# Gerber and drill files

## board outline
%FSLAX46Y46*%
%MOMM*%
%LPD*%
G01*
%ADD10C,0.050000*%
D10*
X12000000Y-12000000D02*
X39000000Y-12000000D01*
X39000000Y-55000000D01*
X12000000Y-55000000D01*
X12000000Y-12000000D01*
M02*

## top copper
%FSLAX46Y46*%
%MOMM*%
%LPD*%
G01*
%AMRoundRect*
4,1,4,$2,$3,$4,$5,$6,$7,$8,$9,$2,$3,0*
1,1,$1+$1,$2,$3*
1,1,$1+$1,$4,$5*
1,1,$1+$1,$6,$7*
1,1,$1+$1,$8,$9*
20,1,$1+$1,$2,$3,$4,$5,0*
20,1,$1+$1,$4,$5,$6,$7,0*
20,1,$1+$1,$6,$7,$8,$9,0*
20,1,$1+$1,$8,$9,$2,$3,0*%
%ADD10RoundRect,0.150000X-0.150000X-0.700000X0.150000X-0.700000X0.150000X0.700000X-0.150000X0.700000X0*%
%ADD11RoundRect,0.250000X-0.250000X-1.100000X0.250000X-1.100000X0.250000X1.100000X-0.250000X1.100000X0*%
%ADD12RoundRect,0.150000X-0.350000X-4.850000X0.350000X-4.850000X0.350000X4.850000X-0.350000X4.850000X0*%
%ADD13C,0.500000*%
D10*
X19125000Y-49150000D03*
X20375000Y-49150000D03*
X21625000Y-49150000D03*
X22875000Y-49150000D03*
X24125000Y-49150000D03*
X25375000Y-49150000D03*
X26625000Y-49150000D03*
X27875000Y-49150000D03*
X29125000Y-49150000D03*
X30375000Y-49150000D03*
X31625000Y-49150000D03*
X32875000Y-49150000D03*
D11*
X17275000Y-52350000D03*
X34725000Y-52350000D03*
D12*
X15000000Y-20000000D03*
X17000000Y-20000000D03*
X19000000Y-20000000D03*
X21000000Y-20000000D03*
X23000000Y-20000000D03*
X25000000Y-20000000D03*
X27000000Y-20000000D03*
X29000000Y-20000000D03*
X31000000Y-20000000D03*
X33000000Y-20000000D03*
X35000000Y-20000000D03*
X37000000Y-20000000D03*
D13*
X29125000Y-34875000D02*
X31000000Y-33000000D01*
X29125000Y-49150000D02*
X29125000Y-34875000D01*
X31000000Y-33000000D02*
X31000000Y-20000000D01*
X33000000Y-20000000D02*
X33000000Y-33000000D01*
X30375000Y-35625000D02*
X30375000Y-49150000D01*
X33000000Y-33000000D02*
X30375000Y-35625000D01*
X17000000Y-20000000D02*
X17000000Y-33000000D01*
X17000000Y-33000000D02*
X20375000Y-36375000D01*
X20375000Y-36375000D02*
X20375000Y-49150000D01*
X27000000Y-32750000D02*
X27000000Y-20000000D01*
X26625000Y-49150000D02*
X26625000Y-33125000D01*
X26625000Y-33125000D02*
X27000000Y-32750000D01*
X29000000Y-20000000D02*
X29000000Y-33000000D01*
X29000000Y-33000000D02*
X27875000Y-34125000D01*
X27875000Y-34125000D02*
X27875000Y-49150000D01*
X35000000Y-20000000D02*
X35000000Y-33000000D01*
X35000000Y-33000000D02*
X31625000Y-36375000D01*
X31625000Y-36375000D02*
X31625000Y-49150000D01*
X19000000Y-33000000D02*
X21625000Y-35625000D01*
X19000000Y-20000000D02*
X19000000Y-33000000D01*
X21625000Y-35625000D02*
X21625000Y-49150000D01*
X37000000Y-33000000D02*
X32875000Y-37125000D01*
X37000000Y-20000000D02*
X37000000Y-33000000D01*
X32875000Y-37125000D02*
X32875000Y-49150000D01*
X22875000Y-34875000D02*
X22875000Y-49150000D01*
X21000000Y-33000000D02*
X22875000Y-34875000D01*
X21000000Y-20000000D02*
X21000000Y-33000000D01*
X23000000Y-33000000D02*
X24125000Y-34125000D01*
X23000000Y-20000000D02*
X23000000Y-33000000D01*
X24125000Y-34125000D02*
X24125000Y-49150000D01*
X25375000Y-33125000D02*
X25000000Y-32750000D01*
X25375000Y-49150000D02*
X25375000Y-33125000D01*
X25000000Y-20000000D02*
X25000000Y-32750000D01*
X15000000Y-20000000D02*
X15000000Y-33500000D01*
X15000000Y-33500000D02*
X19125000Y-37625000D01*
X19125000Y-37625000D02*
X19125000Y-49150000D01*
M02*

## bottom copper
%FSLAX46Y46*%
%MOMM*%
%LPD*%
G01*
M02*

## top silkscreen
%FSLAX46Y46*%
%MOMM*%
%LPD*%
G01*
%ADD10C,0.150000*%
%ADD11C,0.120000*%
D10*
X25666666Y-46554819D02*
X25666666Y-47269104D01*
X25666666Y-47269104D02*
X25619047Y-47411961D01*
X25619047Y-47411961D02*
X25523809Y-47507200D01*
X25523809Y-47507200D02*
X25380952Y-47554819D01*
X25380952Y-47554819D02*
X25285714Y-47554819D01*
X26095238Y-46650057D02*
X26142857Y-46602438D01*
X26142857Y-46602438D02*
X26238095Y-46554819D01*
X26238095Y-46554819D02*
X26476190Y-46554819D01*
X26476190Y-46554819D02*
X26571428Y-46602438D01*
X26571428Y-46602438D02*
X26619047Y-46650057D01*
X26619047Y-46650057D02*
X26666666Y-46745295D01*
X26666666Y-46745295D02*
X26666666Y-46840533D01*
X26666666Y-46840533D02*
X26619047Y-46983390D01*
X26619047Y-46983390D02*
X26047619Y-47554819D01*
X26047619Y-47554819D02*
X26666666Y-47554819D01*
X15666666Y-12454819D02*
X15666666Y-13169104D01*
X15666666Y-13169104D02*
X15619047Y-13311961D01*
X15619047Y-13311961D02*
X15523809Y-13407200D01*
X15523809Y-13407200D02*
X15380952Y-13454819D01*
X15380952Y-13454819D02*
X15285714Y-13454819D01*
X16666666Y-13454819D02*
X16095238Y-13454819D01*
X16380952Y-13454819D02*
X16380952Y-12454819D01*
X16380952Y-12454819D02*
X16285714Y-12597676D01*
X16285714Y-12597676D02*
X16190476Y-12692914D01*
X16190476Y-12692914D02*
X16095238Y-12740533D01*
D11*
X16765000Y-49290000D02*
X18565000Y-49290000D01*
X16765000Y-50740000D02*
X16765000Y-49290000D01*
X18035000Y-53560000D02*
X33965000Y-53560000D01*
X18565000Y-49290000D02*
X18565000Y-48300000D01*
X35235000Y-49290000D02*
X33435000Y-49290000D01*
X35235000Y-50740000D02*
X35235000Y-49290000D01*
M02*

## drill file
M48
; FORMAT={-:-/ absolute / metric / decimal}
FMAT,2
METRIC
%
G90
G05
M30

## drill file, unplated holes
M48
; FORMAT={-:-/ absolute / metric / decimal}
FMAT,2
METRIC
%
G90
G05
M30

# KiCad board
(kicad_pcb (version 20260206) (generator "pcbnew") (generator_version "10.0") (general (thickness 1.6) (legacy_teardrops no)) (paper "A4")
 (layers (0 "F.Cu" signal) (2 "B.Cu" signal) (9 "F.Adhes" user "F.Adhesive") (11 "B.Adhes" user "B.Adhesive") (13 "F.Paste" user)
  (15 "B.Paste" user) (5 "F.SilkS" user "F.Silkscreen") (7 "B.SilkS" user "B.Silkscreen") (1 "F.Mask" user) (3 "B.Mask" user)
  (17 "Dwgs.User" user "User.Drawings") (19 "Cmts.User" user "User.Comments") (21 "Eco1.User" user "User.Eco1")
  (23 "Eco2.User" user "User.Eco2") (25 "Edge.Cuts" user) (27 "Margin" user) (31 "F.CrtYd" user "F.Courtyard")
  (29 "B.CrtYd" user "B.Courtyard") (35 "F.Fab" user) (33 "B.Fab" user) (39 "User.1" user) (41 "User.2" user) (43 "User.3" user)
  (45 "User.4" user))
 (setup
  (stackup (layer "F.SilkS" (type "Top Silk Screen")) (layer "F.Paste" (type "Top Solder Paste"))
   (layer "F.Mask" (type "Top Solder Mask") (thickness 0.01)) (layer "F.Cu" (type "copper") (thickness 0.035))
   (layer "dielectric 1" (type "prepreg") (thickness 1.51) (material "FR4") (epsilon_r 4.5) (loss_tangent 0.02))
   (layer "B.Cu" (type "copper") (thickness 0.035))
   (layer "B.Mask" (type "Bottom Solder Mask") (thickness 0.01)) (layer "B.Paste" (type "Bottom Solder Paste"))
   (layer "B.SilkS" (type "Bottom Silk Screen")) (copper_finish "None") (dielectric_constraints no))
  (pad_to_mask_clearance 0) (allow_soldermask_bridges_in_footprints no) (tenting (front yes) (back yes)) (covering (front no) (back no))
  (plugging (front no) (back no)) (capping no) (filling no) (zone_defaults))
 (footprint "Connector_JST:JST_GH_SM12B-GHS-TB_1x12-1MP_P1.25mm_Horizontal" (layer "F.Cu") (at 26 51)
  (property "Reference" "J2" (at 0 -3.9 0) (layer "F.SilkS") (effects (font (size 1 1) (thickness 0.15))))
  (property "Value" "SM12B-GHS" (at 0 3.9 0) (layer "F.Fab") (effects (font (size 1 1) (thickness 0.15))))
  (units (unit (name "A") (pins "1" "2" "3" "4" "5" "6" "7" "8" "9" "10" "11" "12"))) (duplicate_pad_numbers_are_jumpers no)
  (fp_line (start -9.235 -1.71) (end -7.435 -1.71) (stroke (width 0.12) (type solid)) (layer "F.SilkS"))
  (fp_line (start -9.235 -0.26) (end -9.235 -1.71) (stroke (width 0.12) (type solid)) (layer "F.SilkS"))
  (fp_line (start -7.965 2.56) (end 7.965 2.56) (stroke (width 0.12) (type solid)) (layer "F.SilkS"))
  (fp_line (start -7.435 -1.71) (end -7.435 -2.7) (stroke (width 0.12) (type solid)) (layer "F.SilkS"))
  (fp_line (start 9.235 -1.71) (end 7.435 -1.71) (stroke (width 0.12) (type solid)) (layer "F.SilkS"))
  (fp_line (start 9.235 -0.26) (end 9.235 -1.71) (stroke (width 0.12) (type solid)) (layer "F.SilkS"))
  (pad "1" smd roundrect (at -6.875 -1.85) (size 0.6 1.7) (layers "F.Cu" "F.Mask" "F.Paste") (roundrect_rratio 0.25) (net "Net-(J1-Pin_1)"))
  (pad "2" smd roundrect (at -5.625 -1.85) (size 0.6 1.7) (layers "F.Cu" "F.Mask" "F.Paste") (roundrect_rratio 0.25) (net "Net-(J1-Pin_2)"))
  (pad "3" smd roundrect (at -4.375 -1.85) (size 0.6 1.7) (layers "F.Cu" "F.Mask" "F.Paste") (roundrect_rratio 0.25) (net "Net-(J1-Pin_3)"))
  (pad "4" smd roundrect (at -3.125 -1.85) (size 0.6 1.7) (layers "F.Cu" "F.Mask" "F.Paste") (roundrect_rratio 0.25) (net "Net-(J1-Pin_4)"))
  (pad "5" smd roundrect (at -1.875 -1.85) (size 0.6 1.7) (layers "F.Cu" "F.Mask" "F.Paste") (roundrect_rratio 0.25) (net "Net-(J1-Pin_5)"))
  (pad "6" smd roundrect (at -0.625 -1.85) (size 0.6 1.7) (layers "F.Cu" "F.Mask" "F.Paste") (roundrect_rratio 0.25) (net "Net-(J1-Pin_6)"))
  (pad "7" smd roundrect (at 0.625 -1.85) (size 0.6 1.7) (layers "F.Cu" "F.Mask" "F.Paste") (roundrect_rratio 0.25) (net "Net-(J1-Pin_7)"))
  (pad "8" smd roundrect (at 1.875 -1.85) (size 0.6 1.7) (layers "F.Cu" "F.Mask" "F.Paste") (roundrect_rratio 0.25) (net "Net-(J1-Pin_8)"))
  (pad "9" smd roundrect (at 3.125 -1.85) (size 0.6 1.7) (layers "F.Cu" "F.Mask" "F.Paste") (roundrect_rratio 0.25) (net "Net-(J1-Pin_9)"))
  (pad "10" smd roundrect (at 4.375 -1.85) (size 0.6 1.7) (layers "F.Cu" "F.Mask" "F.Paste") (roundrect_rratio 0.25) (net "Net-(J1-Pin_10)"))
  (pad "11" smd roundrect (at 5.625 -1.85) (size 0.6 1.7) (layers "F.Cu" "F.Mask" "F.Paste") (roundrect_rratio 0.25) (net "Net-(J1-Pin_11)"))
  (pad "12" smd roundrect (at 6.875 -1.85) (size 0.6 1.7) (layers "F.Cu" "F.Mask" "F.Paste") (roundrect_rratio 0.25) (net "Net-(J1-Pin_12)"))
  (pad "MP" smd roundrect (at -8.725 1.35) (size 1 2.7) (layers "F.Cu" "F.Mask" "F.Paste") (roundrect_rratio 0.25))
  (pad "MP" smd roundrect (at 8.725 1.35) (size 1 2.7) (layers "F.Cu" "F.Mask" "F.Paste") (roundrect_rratio 0.25)))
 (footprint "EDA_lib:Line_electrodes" (layer "F.Cu") (at 26 20)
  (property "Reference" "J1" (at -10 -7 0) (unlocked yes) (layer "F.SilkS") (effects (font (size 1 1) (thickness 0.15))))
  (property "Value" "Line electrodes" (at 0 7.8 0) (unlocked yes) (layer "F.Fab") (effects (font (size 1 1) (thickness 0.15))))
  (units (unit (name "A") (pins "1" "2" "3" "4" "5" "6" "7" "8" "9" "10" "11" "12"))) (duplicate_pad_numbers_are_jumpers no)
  (pad "1" smd roundrect (at -11 0) (size 1 10) (layers "F.Cu" "F.Mask" "F.Paste") (roundrect_rratio 0.15) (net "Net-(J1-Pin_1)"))
  (pad "2" smd roundrect (at -9 0) (size 1 10) (layers "F.Cu" "F.Mask" "F.Paste") (roundrect_rratio 0.15) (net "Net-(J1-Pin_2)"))
  (pad "3" smd roundrect (at -7 0) (size 1 10) (layers "F.Cu" "F.Mask" "F.Paste") (roundrect_rratio 0.15) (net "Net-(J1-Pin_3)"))
  (pad "4" smd roundrect (at -5 0) (size 1 10) (layers "F.Cu" "F.Mask" "F.Paste") (roundrect_rratio 0.15) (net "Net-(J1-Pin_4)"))
  (pad "5" smd roundrect (at -3 0) (size 1 10) (layers "F.Cu" "F.Mask" "F.Paste") (roundrect_rratio 0.15) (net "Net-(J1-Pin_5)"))
  (pad "6" smd roundrect (at -1 0) (size 1 10) (layers "F.Cu" "F.Mask" "F.Paste") (roundrect_rratio 0.15) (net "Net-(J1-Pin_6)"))
  (pad "7" smd roundrect (at 1 0) (size 1 10) (layers "F.Cu" "F.Mask" "F.Paste") (roundrect_rratio 0.15) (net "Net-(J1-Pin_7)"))
  (pad "8" smd roundrect (at 3 0) (size 1 10) (layers "F.Cu" "F.Mask" "F.Paste") (roundrect_rratio 0.15) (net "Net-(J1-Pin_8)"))
  (pad "9" smd roundrect (at 5 0) (size 1 10) (layers "F.Cu" "F.Mask" "F.Paste") (roundrect_rratio 0.15) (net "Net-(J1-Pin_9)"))
  (pad "10" smd roundrect (at 7 0) (size 1 10) (layers "F.Cu" "F.Mask" "F.Paste") (roundrect_rratio 0.15) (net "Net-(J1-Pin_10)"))
  (pad "11" smd roundrect (at 9 0) (size 1 10) (layers "F.Cu" "F.Mask" "F.Paste") (roundrect_rratio 0.15) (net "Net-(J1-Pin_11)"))
  (pad "12" smd roundrect (at 11 0) (size 1 10) (layers "F.Cu" "F.Mask" "F.Paste") (roundrect_rratio 0.15) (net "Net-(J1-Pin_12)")))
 (gr_rect (start 12 12) (end 39 55) (stroke (width 0.05) (type default)) (fill no) (layer "Edge.Cuts"))
 (segment (start 29.125 34.875) (end 31 33) (width 0.5) (layer "F.Cu") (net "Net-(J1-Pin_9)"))
 (segment (start 29.125 49.15) (end 29.125 34.875) (width 0.5) (layer "F.Cu") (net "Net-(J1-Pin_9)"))
 (segment (start 31 33) (end 31 20) (width 0.5) (layer "F.Cu") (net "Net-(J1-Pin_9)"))
 (segment (start 33 20) (end 33 33) (width 0.5) (layer "F.Cu") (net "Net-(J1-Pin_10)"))
 (segment (start 30.375 35.625) (end 30.375 49.15) (width 0.5) (layer "F.Cu") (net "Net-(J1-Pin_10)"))
 (segment (start 33 33) (end 30.375 35.625) (width 0.5) (layer "F.Cu") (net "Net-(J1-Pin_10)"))
 (segment (start 17 20) (end 17 33) (width 0.5) (layer "F.Cu") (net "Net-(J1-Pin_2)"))
 (segment (start 17 33) (end 20.375 36.375) (width 0.5) (layer "F.Cu") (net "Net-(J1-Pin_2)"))
 (segment (start 20.375 36.375) (end 20.375 49.15) (width 0.5) (layer "F.Cu") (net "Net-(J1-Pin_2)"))
 (segment (start 27 32.75) (end 27 20) (width 0.5) (layer "F.Cu") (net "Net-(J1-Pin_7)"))
 (segment (start 26.625 49.15) (end 26.625 33.125) (width 0.5) (layer "F.Cu") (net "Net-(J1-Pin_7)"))
 (segment (start 26.625 33.125) (end 27 32.75) (width 0.5) (layer "F.Cu") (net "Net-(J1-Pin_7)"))
 (segment (start 29 20) (end 29 33) (width 0.5) (layer "F.Cu") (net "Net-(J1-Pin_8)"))
 (segment (start 29 33) (end 27.875 34.125) (width 0.5) (layer "F.Cu") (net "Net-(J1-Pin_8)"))
 (segment (start 27.875 34.125) (end 27.875 49.15) (width 0.5) (layer "F.Cu") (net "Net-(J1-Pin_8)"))
 (segment (start 35 20) (end 35 33) (width 0.5) (layer "F.Cu") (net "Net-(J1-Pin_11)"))
 (segment (start 35 33) (end 31.625 36.375) (width 0.5) (layer "F.Cu") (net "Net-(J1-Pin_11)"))
 (segment (start 31.625 36.375) (end 31.625 49.15) (width 0.5) (layer "F.Cu") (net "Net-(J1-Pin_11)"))
 (segment (start 19 33) (end 21.625 35.625) (width 0.5) (layer "F.Cu") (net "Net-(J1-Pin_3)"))
 (segment (start 19 20) (end 19 33) (width 0.5) (layer "F.Cu") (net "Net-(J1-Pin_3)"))
 (segment (start 21.625 35.625) (end 21.625 49.15) (width 0.5) (layer "F.Cu") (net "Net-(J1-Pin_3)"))
 (segment (start 37 33) (end 32.875 37.125) (width 0.5) (layer "F.Cu") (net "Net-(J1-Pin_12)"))
 (segment (start 37 20) (end 37 33) (width 0.5) (layer "F.Cu") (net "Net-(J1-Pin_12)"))
 (segment (start 32.875 37.125) (end 32.875 49.15) (width 0.5) (layer "F.Cu") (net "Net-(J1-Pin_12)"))
 (segment (start 22.875 34.875) (end 22.875 49.15) (width 0.5) (layer "F.Cu") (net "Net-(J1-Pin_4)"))
 (segment (start 21 33) (end 22.875 34.875) (width 0.5) (layer "F.Cu") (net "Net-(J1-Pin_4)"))
 (segment (start 21 20) (end 21 33) (width 0.5) (layer "F.Cu") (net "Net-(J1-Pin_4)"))
 (segment (start 23 33) (end 24.125 34.125) (width 0.5) (layer "F.Cu") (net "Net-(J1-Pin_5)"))
 (segment (start 23 20) (end 23 33) (width 0.5) (layer "F.Cu") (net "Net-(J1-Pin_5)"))
 (segment (start 24.125 34.125) (end 24.125 49.15) (width 0.5) (layer "F.Cu") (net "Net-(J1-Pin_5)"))
 (segment (start 25.375 33.125) (end 25 32.75) (width 0.5) (layer "F.Cu") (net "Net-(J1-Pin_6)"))
 (segment (start 25.375 49.15) (end 25.375 33.125) (width 0.5) (layer "F.Cu") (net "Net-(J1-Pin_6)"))
 (segment (start 25 20) (end 25 32.75) (width 0.5) (layer "F.Cu") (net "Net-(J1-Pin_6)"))
 (segment (start 15 20) (end 15 33.5) (width 0.5) (layer "F.Cu") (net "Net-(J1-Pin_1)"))
 (segment (start 15 33.5) (end 19.125 37.625) (width 0.5) (layer "F.Cu") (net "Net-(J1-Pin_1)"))
 (segment (start 19.125 37.625) (end 19.125 49.15) (width 0.5) (layer "F.Cu") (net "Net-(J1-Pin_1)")))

